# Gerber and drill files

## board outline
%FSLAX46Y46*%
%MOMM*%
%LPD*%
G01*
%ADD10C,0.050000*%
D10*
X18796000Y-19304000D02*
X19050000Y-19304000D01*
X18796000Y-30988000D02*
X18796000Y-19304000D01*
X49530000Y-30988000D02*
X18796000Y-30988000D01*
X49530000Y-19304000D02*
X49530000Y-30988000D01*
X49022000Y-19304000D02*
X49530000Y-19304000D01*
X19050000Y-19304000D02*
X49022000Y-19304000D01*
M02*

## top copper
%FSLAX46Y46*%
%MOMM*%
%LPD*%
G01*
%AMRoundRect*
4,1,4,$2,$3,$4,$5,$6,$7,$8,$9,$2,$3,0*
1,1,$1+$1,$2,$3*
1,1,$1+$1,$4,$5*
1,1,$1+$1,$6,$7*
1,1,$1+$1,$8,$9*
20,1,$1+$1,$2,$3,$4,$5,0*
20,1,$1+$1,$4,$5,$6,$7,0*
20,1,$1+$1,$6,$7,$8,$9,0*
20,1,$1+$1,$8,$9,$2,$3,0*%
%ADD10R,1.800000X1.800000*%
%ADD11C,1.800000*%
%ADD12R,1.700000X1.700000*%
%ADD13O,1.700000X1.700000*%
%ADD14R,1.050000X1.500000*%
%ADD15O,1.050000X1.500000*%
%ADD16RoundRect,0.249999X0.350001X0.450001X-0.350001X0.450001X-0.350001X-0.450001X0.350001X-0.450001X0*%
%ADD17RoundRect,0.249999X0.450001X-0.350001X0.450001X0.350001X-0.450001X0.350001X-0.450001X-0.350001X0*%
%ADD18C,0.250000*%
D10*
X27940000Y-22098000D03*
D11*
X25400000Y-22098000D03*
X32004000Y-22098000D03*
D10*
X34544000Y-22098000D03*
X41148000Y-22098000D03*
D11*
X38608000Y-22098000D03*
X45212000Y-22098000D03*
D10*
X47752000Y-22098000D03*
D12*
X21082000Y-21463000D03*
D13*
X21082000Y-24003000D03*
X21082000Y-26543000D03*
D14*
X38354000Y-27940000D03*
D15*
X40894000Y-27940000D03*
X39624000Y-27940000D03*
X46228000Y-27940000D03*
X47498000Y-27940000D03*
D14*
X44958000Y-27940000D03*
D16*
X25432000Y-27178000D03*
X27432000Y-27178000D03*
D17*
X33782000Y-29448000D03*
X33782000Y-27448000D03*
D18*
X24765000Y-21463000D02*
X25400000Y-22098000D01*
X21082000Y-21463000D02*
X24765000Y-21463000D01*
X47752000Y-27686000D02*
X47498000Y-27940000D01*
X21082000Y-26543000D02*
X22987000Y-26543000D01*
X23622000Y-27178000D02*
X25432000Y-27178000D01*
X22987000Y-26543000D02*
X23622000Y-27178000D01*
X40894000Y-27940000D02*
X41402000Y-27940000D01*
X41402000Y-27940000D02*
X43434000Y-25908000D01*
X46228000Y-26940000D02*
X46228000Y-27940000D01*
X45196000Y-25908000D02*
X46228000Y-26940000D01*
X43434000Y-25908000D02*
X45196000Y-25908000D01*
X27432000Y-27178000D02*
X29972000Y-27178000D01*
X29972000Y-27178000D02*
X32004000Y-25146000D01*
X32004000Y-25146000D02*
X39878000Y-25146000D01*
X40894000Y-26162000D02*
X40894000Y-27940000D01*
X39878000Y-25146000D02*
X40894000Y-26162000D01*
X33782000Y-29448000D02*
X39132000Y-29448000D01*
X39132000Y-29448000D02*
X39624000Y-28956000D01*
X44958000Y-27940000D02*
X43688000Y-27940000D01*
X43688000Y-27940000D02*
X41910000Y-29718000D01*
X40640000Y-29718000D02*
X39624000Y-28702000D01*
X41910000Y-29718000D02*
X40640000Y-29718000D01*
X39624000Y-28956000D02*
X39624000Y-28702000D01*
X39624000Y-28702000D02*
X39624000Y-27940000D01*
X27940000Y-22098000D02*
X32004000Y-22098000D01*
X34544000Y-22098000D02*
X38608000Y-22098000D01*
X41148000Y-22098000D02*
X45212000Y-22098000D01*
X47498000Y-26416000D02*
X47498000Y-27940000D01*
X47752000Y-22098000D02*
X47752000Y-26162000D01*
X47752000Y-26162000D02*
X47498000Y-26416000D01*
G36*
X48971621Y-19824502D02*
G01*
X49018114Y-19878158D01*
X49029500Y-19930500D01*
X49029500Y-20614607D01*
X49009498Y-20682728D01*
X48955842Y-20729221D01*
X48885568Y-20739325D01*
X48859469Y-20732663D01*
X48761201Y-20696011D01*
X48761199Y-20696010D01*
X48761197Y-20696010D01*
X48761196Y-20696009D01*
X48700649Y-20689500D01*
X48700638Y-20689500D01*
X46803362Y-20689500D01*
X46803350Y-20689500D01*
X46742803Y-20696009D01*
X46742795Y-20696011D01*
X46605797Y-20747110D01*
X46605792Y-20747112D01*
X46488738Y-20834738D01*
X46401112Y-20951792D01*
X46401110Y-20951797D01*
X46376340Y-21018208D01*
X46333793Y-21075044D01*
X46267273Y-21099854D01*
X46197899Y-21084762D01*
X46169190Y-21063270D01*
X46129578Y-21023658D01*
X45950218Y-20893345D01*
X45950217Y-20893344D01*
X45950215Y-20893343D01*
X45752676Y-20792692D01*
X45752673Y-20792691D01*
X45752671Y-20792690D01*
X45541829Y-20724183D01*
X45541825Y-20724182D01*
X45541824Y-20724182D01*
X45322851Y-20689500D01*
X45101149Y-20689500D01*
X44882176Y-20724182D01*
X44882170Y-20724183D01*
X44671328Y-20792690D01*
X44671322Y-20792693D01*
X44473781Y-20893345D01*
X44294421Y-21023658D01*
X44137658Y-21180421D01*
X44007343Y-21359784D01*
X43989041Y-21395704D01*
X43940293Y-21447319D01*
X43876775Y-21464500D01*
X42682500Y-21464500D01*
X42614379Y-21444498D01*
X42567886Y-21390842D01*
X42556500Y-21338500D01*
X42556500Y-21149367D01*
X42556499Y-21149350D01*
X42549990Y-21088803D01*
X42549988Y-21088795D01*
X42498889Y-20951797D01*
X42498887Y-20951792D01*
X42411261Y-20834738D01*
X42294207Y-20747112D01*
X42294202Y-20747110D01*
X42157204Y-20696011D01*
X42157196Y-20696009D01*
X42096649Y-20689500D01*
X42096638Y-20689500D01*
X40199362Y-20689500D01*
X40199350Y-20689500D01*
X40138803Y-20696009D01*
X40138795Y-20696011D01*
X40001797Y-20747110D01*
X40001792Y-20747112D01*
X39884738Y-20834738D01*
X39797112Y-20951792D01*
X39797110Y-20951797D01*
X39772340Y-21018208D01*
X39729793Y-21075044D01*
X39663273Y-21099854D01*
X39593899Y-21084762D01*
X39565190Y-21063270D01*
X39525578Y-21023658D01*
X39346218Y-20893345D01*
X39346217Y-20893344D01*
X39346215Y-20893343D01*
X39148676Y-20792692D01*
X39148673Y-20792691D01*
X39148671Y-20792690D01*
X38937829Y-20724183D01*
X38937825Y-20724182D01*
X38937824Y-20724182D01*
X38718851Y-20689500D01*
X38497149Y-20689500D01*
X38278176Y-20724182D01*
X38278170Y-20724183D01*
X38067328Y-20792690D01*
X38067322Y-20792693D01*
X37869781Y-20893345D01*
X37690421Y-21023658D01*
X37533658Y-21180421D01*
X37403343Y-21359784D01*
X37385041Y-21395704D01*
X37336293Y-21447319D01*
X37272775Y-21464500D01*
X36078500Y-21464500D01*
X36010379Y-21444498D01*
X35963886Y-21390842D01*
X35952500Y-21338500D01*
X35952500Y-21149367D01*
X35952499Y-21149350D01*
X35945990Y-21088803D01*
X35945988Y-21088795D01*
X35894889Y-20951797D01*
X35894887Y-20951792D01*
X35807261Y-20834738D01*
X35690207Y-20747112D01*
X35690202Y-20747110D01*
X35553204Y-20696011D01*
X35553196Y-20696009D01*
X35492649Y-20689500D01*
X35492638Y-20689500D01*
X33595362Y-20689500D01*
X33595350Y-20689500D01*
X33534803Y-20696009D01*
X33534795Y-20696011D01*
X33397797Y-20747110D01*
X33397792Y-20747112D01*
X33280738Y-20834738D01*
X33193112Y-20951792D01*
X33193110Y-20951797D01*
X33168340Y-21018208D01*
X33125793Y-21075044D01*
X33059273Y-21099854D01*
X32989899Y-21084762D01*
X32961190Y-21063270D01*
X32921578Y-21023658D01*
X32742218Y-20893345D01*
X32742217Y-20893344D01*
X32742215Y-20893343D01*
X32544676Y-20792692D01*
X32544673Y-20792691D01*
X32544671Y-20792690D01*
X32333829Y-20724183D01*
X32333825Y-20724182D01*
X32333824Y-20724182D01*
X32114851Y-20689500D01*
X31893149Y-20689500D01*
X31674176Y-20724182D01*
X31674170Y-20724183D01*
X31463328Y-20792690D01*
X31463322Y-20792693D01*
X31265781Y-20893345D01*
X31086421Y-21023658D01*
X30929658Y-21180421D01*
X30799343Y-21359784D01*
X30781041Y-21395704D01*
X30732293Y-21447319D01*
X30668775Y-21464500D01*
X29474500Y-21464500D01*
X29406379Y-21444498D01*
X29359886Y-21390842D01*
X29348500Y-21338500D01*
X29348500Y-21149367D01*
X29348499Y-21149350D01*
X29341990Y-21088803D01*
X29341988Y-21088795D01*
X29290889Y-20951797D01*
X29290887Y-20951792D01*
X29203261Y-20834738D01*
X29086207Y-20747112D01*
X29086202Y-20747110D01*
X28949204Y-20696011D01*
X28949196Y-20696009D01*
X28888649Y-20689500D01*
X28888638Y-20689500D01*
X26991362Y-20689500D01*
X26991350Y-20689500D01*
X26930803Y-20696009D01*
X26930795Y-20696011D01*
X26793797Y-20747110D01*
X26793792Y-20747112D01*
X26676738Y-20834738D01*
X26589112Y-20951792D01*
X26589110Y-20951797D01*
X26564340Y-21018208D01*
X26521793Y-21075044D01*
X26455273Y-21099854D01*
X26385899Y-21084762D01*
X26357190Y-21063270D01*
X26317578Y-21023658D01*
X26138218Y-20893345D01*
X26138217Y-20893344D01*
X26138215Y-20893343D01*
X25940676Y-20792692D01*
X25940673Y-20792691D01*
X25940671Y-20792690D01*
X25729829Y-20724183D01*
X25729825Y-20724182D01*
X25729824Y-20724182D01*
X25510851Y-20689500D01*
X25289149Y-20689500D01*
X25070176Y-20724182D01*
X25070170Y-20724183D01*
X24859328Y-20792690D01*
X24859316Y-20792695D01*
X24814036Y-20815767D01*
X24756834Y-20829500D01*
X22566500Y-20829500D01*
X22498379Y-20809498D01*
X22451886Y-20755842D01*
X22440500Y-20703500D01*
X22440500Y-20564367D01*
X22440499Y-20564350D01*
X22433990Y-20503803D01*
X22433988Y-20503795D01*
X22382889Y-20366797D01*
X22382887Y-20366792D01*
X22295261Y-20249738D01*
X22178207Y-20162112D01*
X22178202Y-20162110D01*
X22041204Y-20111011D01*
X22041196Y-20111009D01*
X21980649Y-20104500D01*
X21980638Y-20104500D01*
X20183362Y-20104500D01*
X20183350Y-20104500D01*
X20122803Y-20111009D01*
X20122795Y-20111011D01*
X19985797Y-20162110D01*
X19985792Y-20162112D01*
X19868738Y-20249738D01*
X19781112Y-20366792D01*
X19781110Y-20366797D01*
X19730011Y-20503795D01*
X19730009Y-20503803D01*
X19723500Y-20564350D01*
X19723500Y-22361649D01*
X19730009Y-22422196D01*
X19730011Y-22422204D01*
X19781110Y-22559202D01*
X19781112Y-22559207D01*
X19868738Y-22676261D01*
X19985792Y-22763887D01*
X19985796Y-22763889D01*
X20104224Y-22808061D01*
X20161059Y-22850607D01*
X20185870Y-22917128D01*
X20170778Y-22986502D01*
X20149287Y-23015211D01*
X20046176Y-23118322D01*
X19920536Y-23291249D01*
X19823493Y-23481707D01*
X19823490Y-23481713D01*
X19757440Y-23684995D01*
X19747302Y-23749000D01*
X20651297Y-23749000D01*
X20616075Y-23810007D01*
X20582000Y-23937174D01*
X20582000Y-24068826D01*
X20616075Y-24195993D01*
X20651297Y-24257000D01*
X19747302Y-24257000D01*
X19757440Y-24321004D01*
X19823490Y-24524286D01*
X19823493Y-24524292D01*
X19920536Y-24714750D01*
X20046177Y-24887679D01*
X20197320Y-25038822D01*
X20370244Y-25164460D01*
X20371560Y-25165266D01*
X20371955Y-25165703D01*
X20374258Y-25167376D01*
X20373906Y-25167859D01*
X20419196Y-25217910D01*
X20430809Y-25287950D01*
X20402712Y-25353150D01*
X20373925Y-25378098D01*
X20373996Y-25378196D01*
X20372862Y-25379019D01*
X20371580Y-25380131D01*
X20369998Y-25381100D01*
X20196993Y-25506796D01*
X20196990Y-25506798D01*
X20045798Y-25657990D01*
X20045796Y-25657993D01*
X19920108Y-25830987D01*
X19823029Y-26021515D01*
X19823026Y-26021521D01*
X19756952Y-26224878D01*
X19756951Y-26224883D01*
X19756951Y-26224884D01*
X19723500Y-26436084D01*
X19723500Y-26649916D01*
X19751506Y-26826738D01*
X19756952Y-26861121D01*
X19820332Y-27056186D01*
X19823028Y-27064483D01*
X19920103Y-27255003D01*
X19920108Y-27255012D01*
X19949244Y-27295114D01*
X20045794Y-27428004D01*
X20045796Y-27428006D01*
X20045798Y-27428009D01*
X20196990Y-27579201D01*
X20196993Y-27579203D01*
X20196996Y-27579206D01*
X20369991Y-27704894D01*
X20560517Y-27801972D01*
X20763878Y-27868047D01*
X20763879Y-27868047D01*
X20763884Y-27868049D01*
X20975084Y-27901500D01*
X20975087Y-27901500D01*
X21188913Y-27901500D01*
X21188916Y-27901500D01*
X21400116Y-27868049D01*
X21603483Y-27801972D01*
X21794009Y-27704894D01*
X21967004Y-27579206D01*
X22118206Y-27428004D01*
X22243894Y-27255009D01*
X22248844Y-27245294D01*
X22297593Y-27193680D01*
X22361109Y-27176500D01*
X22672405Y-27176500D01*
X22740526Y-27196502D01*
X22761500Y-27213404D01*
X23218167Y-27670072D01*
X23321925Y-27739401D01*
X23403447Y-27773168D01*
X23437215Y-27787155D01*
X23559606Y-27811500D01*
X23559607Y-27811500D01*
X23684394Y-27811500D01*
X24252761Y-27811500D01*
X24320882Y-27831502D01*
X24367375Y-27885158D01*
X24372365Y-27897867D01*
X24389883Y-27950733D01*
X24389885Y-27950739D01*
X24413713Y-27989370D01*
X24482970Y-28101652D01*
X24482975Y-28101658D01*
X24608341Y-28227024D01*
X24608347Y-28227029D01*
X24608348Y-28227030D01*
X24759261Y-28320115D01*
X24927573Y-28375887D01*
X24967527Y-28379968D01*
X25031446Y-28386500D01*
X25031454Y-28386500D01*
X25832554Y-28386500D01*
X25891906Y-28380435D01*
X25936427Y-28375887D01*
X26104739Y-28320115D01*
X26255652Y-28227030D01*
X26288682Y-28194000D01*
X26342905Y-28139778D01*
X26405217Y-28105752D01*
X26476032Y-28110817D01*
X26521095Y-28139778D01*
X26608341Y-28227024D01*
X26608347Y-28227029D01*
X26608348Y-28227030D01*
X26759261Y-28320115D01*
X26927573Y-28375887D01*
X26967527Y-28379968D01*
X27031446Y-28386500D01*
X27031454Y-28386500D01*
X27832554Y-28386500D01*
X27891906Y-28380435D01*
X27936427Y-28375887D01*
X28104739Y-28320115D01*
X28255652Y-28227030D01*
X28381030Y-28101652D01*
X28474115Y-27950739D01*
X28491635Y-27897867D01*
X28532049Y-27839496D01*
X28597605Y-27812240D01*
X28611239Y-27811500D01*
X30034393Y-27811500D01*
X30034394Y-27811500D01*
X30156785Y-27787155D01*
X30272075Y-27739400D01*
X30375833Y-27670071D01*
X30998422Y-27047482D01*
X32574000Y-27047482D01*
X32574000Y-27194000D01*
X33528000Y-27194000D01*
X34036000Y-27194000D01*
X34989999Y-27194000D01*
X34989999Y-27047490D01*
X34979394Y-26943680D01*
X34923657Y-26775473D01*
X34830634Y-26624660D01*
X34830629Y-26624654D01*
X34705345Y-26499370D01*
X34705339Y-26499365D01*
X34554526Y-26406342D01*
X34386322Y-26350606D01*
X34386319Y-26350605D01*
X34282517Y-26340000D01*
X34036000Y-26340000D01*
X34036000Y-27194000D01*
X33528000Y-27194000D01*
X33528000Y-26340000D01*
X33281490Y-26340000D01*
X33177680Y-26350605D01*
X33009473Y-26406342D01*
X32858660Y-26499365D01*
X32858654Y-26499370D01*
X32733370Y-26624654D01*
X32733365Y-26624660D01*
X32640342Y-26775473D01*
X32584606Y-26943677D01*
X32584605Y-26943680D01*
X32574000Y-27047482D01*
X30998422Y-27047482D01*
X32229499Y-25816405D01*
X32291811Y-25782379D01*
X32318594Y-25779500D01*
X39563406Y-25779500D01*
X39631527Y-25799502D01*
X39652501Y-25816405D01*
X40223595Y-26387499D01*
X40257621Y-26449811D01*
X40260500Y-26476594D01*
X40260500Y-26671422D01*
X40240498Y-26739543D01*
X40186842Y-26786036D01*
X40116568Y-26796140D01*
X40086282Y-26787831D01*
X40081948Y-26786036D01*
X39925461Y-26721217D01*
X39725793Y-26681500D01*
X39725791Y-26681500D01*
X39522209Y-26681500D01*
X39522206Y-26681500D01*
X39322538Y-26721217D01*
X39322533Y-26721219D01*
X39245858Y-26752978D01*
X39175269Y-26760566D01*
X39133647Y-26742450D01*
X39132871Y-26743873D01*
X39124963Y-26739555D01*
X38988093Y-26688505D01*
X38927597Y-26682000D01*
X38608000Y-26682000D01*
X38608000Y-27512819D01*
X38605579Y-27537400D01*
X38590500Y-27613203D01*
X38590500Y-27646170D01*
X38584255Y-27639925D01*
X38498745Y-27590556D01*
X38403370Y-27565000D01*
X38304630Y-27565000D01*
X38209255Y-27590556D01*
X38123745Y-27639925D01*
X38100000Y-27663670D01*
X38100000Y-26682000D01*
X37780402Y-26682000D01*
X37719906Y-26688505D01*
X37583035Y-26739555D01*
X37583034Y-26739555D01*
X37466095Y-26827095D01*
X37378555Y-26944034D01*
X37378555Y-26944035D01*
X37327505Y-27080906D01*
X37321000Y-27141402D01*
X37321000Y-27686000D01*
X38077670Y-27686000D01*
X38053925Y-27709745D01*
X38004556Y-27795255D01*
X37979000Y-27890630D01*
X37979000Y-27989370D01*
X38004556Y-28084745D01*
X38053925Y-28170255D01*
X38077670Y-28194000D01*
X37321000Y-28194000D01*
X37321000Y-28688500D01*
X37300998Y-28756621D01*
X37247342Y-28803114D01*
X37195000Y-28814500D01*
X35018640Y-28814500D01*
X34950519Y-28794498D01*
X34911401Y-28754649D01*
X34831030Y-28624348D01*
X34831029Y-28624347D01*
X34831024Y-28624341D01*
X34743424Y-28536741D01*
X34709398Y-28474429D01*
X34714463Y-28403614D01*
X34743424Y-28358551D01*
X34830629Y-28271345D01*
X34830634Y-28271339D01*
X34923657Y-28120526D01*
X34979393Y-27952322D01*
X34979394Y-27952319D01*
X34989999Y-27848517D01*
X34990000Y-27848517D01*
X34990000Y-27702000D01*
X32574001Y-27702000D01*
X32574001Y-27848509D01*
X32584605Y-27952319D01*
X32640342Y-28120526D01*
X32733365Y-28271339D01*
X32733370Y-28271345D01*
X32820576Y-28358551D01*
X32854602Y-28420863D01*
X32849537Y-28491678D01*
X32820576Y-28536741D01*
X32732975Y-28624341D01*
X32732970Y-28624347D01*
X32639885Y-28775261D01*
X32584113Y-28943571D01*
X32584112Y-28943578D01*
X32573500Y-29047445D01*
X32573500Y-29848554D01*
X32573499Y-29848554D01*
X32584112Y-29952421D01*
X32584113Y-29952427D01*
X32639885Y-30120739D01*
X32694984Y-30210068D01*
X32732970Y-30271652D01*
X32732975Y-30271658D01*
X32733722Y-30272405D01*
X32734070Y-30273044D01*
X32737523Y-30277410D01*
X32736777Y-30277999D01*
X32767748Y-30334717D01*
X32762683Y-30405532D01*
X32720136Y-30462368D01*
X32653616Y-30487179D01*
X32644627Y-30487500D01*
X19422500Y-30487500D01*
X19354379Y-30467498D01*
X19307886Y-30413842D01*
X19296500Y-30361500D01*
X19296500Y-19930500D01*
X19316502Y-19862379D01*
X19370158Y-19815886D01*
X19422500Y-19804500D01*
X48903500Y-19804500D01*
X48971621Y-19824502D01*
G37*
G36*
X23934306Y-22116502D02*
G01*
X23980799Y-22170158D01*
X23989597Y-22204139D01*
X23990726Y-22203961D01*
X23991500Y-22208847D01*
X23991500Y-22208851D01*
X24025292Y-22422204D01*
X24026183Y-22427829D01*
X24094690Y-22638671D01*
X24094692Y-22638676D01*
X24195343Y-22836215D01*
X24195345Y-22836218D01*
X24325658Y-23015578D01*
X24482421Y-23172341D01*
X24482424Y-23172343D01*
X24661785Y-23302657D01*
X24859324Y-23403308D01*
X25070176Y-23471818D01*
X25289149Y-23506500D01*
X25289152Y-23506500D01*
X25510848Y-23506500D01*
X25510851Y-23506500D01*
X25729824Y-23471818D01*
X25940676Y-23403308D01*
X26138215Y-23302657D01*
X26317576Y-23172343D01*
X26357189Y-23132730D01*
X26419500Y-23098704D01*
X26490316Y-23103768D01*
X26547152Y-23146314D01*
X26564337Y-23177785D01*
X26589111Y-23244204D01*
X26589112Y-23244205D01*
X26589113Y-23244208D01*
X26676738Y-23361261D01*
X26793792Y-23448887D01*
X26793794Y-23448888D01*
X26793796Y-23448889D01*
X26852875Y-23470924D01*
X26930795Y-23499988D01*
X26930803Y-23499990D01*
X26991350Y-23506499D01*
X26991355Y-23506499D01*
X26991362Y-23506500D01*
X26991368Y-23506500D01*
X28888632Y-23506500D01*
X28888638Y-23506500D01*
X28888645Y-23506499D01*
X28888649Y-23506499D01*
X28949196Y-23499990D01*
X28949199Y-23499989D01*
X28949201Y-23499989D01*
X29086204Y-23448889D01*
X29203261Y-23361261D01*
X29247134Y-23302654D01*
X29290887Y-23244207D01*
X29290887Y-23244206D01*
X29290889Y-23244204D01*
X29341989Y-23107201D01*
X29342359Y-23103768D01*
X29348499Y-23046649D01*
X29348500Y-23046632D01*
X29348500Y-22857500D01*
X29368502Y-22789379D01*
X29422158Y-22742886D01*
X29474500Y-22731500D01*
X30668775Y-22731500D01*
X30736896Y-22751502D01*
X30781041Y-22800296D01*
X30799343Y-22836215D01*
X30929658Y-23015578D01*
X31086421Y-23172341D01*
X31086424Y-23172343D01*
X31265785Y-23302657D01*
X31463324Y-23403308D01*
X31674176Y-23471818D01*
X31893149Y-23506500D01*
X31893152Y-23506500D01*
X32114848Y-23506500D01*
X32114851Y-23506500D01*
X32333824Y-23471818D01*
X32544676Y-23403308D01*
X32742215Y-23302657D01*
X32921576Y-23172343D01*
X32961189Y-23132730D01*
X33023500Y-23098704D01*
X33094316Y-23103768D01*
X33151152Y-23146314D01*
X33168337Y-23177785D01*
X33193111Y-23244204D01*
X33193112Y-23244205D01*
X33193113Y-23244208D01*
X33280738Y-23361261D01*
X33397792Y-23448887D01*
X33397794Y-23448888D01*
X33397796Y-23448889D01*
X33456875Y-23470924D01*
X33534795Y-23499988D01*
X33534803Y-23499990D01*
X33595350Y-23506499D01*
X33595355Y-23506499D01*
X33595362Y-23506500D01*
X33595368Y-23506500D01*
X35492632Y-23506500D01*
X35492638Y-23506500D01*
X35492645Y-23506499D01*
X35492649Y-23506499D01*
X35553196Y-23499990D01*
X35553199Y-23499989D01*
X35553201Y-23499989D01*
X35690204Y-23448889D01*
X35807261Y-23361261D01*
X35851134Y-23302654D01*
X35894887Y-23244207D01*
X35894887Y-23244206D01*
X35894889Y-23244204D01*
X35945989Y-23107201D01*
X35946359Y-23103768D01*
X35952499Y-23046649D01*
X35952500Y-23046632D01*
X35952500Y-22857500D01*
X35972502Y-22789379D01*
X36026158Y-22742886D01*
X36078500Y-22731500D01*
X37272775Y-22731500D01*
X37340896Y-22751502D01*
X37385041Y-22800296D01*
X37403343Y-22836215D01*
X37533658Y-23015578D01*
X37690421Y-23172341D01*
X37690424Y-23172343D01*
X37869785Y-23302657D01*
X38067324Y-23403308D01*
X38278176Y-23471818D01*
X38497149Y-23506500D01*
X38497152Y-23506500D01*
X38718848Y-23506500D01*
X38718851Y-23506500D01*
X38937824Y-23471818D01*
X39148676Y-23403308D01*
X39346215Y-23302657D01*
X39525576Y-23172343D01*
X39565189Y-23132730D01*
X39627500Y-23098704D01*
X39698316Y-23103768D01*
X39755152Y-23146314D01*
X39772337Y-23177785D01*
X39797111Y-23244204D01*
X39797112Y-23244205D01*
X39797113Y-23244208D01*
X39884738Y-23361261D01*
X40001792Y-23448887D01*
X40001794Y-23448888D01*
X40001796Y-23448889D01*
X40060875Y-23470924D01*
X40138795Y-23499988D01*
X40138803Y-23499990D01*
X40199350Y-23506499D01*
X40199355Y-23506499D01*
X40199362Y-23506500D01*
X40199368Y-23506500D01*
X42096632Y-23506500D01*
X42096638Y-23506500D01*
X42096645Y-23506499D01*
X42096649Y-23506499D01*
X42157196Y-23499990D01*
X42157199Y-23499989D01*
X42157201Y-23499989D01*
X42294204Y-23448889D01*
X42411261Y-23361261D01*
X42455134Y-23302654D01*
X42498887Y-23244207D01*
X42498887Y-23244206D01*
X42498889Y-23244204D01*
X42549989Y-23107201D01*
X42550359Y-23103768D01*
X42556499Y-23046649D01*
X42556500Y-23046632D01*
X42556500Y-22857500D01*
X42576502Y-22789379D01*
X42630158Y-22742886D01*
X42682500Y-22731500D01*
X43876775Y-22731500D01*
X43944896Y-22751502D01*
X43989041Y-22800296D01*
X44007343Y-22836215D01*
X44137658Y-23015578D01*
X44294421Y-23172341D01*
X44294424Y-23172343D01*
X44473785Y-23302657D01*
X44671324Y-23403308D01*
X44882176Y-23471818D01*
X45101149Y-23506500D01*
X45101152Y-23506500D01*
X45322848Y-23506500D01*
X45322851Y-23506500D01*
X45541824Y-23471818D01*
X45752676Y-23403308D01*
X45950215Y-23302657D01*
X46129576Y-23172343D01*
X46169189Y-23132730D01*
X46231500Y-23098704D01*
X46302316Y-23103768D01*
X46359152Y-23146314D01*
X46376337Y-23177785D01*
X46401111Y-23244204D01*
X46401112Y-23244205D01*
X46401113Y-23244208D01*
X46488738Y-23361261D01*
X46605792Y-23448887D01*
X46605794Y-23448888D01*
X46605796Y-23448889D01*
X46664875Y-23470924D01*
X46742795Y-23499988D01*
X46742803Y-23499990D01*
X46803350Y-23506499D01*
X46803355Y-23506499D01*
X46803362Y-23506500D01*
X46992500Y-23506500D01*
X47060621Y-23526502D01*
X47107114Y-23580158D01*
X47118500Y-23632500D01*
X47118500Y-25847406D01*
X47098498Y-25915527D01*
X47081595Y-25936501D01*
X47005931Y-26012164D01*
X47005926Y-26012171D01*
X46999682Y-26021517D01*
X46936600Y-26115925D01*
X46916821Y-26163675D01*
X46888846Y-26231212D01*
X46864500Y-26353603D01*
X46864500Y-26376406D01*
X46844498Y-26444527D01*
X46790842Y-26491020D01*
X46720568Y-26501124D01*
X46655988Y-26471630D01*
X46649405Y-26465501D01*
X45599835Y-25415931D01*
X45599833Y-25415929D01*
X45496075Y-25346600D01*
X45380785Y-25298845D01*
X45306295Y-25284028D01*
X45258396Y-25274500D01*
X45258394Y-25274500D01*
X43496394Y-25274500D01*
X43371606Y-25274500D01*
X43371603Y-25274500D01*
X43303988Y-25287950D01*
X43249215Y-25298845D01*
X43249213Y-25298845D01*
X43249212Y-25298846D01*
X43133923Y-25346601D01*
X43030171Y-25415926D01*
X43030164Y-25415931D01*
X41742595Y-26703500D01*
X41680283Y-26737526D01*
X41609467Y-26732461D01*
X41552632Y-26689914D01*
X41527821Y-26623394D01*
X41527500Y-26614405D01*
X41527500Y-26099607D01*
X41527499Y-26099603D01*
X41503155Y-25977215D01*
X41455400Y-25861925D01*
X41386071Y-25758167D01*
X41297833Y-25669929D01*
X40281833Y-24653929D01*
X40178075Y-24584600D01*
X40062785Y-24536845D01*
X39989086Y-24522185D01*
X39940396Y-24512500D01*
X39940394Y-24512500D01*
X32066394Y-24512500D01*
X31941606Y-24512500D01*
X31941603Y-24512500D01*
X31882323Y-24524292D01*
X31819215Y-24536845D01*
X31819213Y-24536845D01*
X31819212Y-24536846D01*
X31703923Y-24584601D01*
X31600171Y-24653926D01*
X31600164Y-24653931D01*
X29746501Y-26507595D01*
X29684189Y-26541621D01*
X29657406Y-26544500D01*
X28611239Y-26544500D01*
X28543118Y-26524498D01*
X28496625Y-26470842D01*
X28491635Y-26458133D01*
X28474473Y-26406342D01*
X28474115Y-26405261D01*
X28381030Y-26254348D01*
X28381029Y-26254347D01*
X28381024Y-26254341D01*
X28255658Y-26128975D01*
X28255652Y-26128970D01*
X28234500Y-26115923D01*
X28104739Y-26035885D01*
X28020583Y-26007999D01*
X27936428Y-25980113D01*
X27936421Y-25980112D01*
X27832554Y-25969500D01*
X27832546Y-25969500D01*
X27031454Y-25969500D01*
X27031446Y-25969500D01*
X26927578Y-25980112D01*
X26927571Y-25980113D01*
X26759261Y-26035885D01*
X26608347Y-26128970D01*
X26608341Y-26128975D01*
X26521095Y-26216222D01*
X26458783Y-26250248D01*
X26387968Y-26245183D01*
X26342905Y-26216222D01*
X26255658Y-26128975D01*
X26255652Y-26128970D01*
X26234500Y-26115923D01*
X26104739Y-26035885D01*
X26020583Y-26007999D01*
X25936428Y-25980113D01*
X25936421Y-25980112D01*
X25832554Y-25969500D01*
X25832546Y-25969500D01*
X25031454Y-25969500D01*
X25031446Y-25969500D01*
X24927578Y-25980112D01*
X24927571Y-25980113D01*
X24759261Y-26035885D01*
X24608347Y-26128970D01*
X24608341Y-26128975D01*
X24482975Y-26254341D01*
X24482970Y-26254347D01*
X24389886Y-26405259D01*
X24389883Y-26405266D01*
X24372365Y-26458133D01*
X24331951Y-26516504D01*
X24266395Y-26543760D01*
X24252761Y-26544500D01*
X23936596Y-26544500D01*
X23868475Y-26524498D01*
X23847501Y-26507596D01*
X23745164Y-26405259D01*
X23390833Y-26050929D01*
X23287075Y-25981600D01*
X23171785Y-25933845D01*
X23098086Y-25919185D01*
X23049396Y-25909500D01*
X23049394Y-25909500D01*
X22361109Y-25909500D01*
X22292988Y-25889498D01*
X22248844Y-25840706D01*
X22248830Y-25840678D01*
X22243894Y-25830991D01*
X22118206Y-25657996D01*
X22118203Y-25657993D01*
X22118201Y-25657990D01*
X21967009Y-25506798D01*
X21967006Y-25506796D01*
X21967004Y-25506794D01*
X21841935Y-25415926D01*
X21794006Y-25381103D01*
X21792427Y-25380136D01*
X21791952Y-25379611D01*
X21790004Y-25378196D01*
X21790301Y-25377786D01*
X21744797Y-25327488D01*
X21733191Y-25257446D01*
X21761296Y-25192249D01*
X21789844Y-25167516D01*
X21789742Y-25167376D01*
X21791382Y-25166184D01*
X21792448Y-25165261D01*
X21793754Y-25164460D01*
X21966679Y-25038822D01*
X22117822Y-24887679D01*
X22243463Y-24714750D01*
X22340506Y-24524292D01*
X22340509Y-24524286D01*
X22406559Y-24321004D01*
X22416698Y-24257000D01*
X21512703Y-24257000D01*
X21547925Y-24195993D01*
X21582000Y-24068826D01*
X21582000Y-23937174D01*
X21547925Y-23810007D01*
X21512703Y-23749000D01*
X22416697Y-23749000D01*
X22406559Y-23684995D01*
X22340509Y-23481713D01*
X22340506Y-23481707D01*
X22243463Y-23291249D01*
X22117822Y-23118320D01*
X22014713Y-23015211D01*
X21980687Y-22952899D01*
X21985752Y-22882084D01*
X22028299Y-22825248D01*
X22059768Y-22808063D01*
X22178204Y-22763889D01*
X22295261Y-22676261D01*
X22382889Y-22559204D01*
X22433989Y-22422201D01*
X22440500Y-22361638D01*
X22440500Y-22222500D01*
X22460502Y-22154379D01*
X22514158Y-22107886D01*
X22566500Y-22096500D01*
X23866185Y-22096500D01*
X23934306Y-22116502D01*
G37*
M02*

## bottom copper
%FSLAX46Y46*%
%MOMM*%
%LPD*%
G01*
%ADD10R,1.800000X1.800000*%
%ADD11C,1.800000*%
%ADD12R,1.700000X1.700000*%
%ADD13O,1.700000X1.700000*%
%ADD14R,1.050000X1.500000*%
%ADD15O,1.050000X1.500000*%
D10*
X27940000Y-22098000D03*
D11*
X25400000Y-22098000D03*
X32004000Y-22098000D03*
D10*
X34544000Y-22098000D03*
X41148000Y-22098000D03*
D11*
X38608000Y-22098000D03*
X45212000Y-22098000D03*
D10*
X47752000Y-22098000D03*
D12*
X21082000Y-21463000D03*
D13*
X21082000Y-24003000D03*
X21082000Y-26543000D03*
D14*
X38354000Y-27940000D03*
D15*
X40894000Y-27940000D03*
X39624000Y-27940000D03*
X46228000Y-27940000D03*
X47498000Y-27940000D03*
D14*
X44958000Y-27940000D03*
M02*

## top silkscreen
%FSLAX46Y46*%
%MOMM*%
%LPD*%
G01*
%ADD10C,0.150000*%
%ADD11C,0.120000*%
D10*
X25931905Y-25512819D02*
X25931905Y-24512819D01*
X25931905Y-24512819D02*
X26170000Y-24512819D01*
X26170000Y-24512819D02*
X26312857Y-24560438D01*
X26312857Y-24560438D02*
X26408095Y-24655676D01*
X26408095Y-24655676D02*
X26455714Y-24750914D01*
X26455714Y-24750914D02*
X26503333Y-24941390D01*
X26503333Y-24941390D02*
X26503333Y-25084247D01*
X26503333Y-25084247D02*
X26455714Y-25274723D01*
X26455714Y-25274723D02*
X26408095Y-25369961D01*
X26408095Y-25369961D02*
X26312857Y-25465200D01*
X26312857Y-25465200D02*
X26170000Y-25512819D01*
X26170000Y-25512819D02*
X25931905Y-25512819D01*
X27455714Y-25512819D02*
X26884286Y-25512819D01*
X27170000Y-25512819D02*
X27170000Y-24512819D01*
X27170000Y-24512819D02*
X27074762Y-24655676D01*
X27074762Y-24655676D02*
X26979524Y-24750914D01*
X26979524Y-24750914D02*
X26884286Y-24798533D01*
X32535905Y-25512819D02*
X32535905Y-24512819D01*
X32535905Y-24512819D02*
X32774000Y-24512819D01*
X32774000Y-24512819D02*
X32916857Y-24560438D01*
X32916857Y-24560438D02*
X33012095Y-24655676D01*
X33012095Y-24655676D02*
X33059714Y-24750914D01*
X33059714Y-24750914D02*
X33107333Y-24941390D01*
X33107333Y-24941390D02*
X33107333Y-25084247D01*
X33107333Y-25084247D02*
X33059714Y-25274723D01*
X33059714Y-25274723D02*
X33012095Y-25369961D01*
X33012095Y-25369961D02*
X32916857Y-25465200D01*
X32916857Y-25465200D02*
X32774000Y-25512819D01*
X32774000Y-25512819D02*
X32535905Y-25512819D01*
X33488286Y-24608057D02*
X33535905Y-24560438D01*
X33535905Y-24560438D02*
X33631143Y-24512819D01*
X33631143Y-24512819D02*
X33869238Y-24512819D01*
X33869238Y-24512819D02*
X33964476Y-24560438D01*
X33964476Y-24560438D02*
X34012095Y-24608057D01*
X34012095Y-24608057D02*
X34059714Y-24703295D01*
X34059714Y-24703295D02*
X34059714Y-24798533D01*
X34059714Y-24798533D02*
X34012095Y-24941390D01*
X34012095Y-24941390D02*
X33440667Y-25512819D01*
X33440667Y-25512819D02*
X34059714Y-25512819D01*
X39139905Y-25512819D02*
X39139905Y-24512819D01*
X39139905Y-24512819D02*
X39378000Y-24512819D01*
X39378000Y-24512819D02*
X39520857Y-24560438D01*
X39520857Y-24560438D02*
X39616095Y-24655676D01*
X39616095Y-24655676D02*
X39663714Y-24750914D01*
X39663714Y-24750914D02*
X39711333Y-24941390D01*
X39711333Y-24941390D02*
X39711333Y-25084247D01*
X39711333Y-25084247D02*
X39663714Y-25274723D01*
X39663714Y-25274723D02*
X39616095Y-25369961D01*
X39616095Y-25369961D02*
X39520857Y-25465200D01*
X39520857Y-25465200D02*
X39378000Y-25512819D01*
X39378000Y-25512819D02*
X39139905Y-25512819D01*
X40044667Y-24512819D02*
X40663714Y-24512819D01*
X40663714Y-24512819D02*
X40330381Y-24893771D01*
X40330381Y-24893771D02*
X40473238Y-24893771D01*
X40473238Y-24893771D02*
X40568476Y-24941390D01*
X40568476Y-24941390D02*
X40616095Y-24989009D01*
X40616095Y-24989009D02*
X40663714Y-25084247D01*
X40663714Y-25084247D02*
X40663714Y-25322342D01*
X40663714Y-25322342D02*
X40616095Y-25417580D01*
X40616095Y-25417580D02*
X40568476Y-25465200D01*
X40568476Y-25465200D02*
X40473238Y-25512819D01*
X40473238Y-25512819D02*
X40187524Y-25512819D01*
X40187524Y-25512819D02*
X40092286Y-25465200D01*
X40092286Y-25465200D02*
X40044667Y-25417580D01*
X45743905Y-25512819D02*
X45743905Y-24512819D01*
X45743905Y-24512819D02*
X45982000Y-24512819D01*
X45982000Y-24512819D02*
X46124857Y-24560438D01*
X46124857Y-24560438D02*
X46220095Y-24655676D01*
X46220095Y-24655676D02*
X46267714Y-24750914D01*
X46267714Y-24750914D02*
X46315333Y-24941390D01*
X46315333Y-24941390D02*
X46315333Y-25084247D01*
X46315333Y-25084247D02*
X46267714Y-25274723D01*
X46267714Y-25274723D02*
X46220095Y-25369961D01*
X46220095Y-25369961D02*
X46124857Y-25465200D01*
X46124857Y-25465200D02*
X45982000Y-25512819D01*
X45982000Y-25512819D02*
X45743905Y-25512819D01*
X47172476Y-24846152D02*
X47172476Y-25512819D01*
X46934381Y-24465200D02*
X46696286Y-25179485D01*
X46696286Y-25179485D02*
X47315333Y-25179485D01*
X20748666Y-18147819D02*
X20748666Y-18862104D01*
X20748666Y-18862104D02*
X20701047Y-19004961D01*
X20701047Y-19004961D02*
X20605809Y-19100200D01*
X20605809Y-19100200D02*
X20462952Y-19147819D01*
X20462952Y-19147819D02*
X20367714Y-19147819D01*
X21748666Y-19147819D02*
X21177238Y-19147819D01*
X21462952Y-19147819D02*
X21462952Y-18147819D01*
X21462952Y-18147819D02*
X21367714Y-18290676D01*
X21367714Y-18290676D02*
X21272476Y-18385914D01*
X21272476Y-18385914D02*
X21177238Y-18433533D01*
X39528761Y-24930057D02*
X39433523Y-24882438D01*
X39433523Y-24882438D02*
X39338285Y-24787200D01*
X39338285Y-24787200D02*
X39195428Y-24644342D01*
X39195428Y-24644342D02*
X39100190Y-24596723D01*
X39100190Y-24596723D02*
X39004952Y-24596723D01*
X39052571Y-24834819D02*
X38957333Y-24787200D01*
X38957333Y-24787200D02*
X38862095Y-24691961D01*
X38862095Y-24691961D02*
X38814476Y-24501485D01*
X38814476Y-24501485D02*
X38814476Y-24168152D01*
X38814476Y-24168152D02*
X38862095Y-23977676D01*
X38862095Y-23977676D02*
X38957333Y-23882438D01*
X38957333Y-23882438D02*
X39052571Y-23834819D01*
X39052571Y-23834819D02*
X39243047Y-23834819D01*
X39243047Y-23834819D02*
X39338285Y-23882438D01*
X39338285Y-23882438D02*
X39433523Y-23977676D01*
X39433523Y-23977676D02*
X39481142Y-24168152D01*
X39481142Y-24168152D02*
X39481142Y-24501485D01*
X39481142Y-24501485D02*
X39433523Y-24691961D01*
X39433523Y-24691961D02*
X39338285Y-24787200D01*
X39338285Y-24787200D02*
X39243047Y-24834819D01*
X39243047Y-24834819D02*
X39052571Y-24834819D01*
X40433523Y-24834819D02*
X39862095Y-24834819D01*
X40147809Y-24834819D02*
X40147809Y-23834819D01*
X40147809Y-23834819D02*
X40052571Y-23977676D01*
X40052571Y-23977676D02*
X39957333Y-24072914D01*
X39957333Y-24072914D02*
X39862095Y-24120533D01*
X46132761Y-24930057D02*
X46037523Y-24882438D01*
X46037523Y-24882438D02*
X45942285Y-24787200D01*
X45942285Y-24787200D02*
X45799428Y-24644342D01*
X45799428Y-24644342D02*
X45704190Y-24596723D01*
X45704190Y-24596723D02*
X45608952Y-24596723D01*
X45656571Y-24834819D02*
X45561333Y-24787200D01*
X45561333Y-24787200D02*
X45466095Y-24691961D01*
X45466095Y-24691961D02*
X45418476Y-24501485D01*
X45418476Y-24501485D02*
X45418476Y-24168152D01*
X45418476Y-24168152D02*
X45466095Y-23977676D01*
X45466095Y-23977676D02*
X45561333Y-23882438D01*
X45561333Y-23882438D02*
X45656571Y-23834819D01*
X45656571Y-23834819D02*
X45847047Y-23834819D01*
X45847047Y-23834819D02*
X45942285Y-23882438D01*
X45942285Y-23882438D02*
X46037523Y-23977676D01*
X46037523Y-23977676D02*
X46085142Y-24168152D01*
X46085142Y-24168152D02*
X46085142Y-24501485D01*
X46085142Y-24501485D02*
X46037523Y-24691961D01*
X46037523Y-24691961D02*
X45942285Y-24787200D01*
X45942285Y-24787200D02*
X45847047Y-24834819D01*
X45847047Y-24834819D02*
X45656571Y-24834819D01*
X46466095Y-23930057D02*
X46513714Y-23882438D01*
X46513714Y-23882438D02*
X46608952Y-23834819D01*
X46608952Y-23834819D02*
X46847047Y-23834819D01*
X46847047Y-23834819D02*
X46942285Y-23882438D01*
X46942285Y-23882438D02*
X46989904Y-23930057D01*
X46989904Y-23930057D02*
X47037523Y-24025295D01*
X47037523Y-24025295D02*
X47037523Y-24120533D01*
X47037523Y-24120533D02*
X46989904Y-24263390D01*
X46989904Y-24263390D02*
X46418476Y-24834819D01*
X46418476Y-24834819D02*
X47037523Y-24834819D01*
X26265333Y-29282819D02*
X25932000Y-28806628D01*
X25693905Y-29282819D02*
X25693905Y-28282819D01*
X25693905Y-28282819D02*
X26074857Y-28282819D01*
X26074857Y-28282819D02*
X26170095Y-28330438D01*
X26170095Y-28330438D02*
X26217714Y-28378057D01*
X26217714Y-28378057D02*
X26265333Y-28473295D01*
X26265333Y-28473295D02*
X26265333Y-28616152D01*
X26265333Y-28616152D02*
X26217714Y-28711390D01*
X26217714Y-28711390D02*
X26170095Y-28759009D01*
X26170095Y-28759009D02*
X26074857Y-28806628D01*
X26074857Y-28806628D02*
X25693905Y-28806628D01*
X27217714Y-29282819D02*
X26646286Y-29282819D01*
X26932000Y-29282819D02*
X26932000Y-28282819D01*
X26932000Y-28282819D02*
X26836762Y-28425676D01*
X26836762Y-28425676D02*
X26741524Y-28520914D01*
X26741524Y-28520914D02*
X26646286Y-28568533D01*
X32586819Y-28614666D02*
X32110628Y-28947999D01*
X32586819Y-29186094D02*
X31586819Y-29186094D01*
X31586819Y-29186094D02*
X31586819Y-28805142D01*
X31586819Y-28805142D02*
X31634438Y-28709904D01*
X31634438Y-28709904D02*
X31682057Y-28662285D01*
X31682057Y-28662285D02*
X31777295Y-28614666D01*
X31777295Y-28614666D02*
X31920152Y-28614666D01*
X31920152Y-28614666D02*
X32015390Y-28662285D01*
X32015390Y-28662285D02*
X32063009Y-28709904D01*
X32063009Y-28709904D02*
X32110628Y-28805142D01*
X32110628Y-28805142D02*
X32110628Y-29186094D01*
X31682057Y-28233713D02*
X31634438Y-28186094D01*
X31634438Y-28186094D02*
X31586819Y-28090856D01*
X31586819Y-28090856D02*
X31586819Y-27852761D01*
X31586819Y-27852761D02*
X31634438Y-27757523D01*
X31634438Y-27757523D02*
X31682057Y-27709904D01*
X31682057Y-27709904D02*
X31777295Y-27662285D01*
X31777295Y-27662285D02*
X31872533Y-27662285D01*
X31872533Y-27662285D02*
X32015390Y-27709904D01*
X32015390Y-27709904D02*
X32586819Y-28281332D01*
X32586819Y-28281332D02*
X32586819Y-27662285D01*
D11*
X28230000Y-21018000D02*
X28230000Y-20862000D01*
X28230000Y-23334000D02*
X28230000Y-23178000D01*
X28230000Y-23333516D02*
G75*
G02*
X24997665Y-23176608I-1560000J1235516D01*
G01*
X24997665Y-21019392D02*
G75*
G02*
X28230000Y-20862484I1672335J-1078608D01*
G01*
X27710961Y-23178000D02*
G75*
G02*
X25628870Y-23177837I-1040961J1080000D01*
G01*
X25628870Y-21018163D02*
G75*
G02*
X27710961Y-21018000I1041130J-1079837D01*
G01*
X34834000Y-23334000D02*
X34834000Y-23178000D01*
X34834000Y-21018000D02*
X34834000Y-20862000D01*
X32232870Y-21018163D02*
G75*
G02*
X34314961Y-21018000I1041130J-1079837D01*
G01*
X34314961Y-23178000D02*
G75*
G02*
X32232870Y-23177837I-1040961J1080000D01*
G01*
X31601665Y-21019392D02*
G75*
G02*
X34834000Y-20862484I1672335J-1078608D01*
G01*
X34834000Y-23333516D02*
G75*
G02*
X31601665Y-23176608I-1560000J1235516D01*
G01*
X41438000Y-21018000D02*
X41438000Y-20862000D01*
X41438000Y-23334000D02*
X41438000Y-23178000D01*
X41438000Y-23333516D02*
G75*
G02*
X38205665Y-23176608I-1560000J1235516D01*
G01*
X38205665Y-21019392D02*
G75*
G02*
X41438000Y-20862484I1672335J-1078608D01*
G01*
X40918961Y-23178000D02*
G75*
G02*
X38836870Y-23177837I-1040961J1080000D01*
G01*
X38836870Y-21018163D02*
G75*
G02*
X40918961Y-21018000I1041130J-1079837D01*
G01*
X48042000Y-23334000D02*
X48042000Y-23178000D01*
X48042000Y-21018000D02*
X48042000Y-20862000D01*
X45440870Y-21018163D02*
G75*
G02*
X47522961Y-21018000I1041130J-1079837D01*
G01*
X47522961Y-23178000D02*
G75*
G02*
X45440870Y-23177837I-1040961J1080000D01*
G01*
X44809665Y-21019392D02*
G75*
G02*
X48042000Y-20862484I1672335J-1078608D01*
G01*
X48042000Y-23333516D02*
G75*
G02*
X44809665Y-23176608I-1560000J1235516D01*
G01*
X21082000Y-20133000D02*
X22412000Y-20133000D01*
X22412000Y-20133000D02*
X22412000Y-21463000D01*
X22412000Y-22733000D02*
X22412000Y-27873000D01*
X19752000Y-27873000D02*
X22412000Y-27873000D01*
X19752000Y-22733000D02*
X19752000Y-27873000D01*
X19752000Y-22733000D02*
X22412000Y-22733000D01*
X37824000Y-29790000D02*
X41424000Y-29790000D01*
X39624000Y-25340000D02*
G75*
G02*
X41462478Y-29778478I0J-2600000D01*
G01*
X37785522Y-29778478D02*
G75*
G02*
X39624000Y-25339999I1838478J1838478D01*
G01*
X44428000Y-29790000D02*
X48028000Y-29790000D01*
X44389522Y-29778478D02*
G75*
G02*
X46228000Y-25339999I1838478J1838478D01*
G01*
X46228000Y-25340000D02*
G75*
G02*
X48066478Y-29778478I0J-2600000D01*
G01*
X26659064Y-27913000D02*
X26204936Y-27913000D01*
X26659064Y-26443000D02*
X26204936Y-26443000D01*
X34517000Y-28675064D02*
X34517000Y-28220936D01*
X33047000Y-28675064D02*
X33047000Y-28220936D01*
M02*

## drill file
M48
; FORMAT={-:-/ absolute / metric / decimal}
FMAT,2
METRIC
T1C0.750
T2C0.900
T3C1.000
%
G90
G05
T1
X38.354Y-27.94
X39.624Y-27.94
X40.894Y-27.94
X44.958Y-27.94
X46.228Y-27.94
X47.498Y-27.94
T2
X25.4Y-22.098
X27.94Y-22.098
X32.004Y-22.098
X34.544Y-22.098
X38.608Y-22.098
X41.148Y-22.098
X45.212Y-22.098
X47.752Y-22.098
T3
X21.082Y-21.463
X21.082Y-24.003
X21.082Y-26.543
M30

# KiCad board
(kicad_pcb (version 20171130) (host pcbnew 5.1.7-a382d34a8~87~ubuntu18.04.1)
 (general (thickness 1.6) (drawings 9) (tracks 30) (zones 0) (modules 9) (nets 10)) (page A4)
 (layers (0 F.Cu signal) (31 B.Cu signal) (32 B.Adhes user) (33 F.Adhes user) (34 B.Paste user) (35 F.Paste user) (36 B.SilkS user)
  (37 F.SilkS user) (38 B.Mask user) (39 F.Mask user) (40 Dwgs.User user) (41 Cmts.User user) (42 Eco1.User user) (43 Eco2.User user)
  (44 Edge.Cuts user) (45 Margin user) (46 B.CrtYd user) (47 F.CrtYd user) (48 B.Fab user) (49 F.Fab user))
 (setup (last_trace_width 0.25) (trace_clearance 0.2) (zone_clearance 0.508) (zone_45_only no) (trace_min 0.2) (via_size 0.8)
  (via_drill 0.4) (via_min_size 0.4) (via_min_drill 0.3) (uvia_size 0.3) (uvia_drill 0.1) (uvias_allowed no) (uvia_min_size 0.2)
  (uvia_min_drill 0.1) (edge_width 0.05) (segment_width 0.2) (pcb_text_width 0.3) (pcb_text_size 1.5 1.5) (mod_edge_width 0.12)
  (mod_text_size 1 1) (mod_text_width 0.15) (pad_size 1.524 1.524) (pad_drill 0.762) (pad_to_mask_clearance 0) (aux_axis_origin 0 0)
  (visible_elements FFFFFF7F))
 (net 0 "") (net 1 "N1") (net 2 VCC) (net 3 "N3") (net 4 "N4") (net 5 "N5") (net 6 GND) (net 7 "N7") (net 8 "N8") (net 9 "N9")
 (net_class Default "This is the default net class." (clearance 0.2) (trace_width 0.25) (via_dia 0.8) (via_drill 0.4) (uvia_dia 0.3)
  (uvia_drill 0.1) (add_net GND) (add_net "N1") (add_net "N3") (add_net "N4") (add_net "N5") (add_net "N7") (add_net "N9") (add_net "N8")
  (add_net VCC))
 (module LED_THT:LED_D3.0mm (layer F.Cu) (at 27.94 22.098 180)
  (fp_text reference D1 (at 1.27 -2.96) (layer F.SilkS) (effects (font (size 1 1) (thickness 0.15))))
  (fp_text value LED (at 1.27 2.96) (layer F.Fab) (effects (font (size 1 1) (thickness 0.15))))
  (fp_line (start -0.29 1.08) (end -0.29 1.236) (layer F.SilkS) (width 0.12))
  (fp_line (start -0.29 -1.236) (end -0.29 -1.08) (layer F.SilkS) (width 0.12))
  (fp_arc (start 1.27 0) (end -0.29 -1.235516) (angle 108.8) (layer F.SilkS) (width 0.12))
  (fp_arc (start 1.27 0) (end -0.29 1.235516) (angle -108.8) (layer F.SilkS) (width 0.12))
  (fp_arc (start 1.27 0) (end 0.229039 -1.08) (angle 87.9) (layer F.SilkS) (width 0.12))
  (fp_arc (start 1.27 0) (end 0.229039 1.08) (angle -87.9) (layer F.SilkS) (width 0.12))
  (pad 1 thru_hole rect (at 0 0 180) (size 1.8 1.8) (drill 0.9) (layers *.Cu *.Mask) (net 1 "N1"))
  (pad 2 thru_hole circle (at 2.54 0 180) (size 1.8 1.8) (drill 0.9) (layers *.Cu *.Mask) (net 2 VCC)))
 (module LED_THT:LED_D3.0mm (layer F.Cu) (at 34.544 22.098 180)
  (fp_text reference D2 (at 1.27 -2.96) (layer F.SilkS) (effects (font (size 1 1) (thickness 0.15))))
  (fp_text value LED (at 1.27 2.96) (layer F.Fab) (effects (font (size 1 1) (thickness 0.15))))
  (fp_line (start -0.29 -1.236) (end -0.29 -1.08) (layer F.SilkS) (width 0.12))
  (fp_line (start -0.29 1.08) (end -0.29 1.236) (layer F.SilkS) (width 0.12))
  (fp_arc (start 1.27 0) (end 0.229039 1.08) (angle -87.9) (layer F.SilkS) (width 0.12))
  (fp_arc (start 1.27 0) (end 0.229039 -1.08) (angle 87.9) (layer F.SilkS) (width 0.12))
  (fp_arc (start 1.27 0) (end -0.29 1.235516) (angle -108.8) (layer F.SilkS) (width 0.12))
  (fp_arc (start 1.27 0) (end -0.29 -1.235516) (angle 108.8) (layer F.SilkS) (width 0.12))
  (pad 2 thru_hole circle (at 2.54 0 180) (size 1.8 1.8) (drill 0.9) (layers *.Cu *.Mask) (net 1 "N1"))
  (pad 1 thru_hole rect (at 0 0 180) (size 1.8 1.8) (drill 0.9) (layers *.Cu *.Mask) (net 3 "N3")))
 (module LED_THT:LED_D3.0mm (layer F.Cu) (at 41.148 22.098 180)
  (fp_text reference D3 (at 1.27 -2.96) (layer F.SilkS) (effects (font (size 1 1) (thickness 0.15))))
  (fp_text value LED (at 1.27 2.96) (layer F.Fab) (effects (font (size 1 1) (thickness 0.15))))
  (fp_line (start -0.29 1.08) (end -0.29 1.236) (layer F.SilkS) (width 0.12))
  (fp_line (start -0.29 -1.236) (end -0.29 -1.08) (layer F.SilkS) (width 0.12))
  (fp_arc (start 1.27 0) (end -0.29 -1.235516) (angle 108.8) (layer F.SilkS) (width 0.12))
  (fp_arc (start 1.27 0) (end -0.29 1.235516) (angle -108.8) (layer F.SilkS) (width 0.12))
  (fp_arc (start 1.27 0) (end 0.229039 -1.08) (angle 87.9) (layer F.SilkS) (width 0.12))
  (fp_arc (start 1.27 0) (end 0.229039 1.08) (angle -87.9) (layer F.SilkS) (width 0.12))
  (pad 1 thru_hole rect (at 0 0 180) (size 1.8 1.8) (drill 0.9) (layers *.Cu *.Mask) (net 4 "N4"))
  (pad 2 thru_hole circle (at 2.54 0 180) (size 1.8 1.8) (drill 0.9) (layers *.Cu *.Mask) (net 3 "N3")))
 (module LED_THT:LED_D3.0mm (layer F.Cu) (at 47.752 22.098 180)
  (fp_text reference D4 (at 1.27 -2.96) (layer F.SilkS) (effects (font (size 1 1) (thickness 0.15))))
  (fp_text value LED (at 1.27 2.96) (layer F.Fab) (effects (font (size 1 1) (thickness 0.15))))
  (fp_line (start -0.29 -1.236) (end -0.29 -1.08) (layer F.SilkS) (width 0.12))
  (fp_line (start -0.29 1.08) (end -0.29 1.236) (layer F.SilkS) (width 0.12))
  (fp_arc (start 1.27 0) (end 0.229039 1.08) (angle -87.9) (layer F.SilkS) (width 0.12))
  (fp_arc (start 1.27 0) (end 0.229039 -1.08) (angle 87.9) (layer F.SilkS) (width 0.12))
  (fp_arc (start 1.27 0) (end -0.29 1.235516) (angle -108.8) (layer F.SilkS) (width 0.12))
  (fp_arc (start 1.27 0) (end -0.29 -1.235516) (angle 108.8) (layer F.SilkS) (width 0.12))
  (pad 2 thru_hole circle (at 2.54 0 180) (size 1.8 1.8) (drill 0.9) (layers *.Cu *.Mask) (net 4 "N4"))
  (pad 1 thru_hole rect (at 0 0 180) (size 1.8 1.8) (drill 0.9) (layers *.Cu *.Mask) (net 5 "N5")))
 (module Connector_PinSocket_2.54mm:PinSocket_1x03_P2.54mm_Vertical (layer F.Cu) (at 21.082 21.463)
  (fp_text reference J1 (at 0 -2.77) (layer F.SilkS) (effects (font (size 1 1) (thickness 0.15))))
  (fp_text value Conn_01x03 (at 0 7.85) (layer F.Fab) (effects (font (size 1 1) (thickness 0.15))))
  (fp_line (start 0 -1.33) (end 1.33 -1.33) (layer F.SilkS) (width 0.12))
  (fp_line (start 1.33 -1.33) (end 1.33 0) (layer F.SilkS) (width 0.12))
  (fp_line (start 1.33 1.27) (end 1.33 6.41) (layer F.SilkS) (width 0.12))
  (fp_line (start -1.33 6.41) (end 1.33 6.41) (layer F.SilkS) (width 0.12))
  (fp_line (start -1.33 1.27) (end -1.33 6.41) (layer F.SilkS) (width 0.12))
  (fp_line (start -1.33 1.27) (end 1.33 1.27) (layer F.SilkS) (width 0.12))
  (pad 1 thru_hole rect (at 0 0) (size 1.7 1.7) (drill 1) (layers *.Cu *.Mask) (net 2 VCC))
  (pad 2 thru_hole oval (at 0 2.54) (size 1.7 1.7) (drill 1) (layers *.Cu *.Mask) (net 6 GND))
  (pad 3 thru_hole oval (at 0 5.08) (size 1.7 1.7) (drill 1) (layers *.Cu *.Mask) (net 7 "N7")))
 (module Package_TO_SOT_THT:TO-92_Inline (layer F.Cu) (at 38.354 27.94)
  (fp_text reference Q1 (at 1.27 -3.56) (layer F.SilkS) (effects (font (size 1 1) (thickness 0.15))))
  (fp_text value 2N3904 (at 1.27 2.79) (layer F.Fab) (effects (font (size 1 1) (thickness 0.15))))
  (fp_line (start -0.53 1.85) (end 3.07 1.85) (layer F.SilkS) (width 0.12))
  (fp_arc (start 1.27 0) (end 1.27 -2.6) (angle 135) (layer F.SilkS) (width 0.12))
  (fp_arc (start 1.27 0) (end 1.27 -2.6) (angle -135) (layer F.SilkS) (width 0.12))
  (pad 1 thru_hole rect (at 0 0) (size 1.05 1.5) (drill 0.75) (layers *.Cu *.Mask) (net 6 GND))
  (pad 3 thru_hole oval (at 2.54 0) (size 1.05 1.5) (drill 0.75) (layers *.Cu *.Mask) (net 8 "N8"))
  (pad 2 thru_hole oval (at 1.27 0) (size 1.05 1.5) (drill 0.75) (layers *.Cu *.Mask) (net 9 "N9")))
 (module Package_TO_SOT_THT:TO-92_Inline (layer F.Cu) (at 44.958 27.94)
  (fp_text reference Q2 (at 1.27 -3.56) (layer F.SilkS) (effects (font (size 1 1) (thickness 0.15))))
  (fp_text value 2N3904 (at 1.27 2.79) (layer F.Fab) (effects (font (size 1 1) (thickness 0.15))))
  (fp_line (start -0.53 1.85) (end 3.07 1.85) (layer F.SilkS) (width 0.12))
  (fp_arc (start 1.27 0) (end 1.27 -2.6) (angle -135) (layer F.SilkS) (width 0.12))
  (fp_arc (start 1.27 0) (end 1.27 -2.6) (angle 135) (layer F.SilkS) (width 0.12))
  (pad 2 thru_hole oval (at 1.27 0) (size 1.05 1.5) (drill 0.75) (layers *.Cu *.Mask) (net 8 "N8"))
  (pad 3 thru_hole oval (at 2.54 0) (size 1.05 1.5) (drill 0.75) (layers *.Cu *.Mask) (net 5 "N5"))
  (pad 1 thru_hole rect (at 0 0) (size 1.05 1.5) (drill 0.75) (layers *.Cu *.Mask) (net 9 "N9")))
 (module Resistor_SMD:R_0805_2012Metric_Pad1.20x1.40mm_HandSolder (layer F.Cu) (at 26.432 27.178 180)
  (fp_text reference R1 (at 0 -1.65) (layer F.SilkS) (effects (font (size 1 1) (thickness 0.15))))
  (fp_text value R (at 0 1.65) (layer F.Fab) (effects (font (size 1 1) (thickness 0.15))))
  (fp_line (start -0.227064 -0.735) (end 0.227064 -0.735) (layer F.SilkS) (width 0.12))
  (fp_line (start -0.227064 0.735) (end 0.227064 0.735) (layer F.SilkS) (width 0.12))
  (pad 2 smd roundrect (at 1 0 180) (size 1.2 1.4) (layers F.Cu F.Paste F.Mask) (roundrect_rratio 0.2083325) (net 7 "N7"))
  (pad 1 smd roundrect (at -1 0 180) (size 1.2 1.4) (layers F.Cu F.Paste F.Mask) (roundrect_rratio 0.2083325) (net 8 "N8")))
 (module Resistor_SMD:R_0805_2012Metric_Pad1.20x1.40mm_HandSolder (layer F.Cu) (at 33.782 28.448 90)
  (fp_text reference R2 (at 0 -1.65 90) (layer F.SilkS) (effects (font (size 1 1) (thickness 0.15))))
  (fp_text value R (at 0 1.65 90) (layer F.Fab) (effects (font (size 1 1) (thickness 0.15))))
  (fp_line (start -0.227064 0.735) (end 0.227064 0.735) (layer F.SilkS) (width 0.12))
  (fp_line (start -0.227064 -0.735) (end 0.227064 -0.735) (layer F.SilkS) (width 0.12))
  (pad 1 smd roundrect (at -1 0 90) (size 1.2 1.4) (layers F.Cu F.Paste F.Mask) (roundrect_rratio 0.2083325) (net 9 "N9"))
  (pad 2 smd roundrect (at 1 0 90) (size 1.2 1.4) (layers F.Cu F.Paste F.Mask) (roundrect_rratio 0.2083325) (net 6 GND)))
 (gr_line (start 18.796 19.304) (end 19.05 19.304) (layer Edge.Cuts) (width 0.05))
 (gr_line (start 18.796 30.988) (end 18.796 19.304) (layer Edge.Cuts) (width 0.05))
 (gr_line (start 49.53 30.988) (end 18.796 30.988) (layer Edge.Cuts) (width 0.05))
 (gr_line (start 49.53 19.304) (end 49.53 30.988) (layer Edge.Cuts) (width 0.05))
 (gr_line (start 49.022 19.304) (end 49.53 19.304) (layer Edge.Cuts) (width 0.05))
 (gr_line (start 19.05 19.304) (end 49.022 19.304) (layer Edge.Cuts) (width 0.05))
 (segment (start 24.765 21.463) (end 25.4 22.098) (width 0.25) (layer F.Cu) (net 2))
 (segment (start 21.082 21.463) (end 24.765 21.463) (width 0.25) (layer F.Cu) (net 2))
 (segment (start 47.752 27.686) (end 47.498 27.94) (width 0.25) (layer F.Cu) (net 5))
 (segment (start 21.082 26.543) (end 22.987 26.543) (width 0.25) (layer F.Cu) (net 7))
 (segment (start 23.622 27.178) (end 25.432 27.178) (width 0.25) (layer F.Cu) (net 7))
 (segment (start 22.987 26.543) (end 23.622 27.178) (width 0.25) (layer F.Cu) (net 7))
 (segment (start 40.894 27.94) (end 41.402 27.94) (width 0.25) (layer F.Cu) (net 8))
 (segment (start 41.402 27.94) (end 43.434 25.908) (width 0.25) (layer F.Cu) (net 8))
 (segment (start 46.228 26.94) (end 46.228 27.94) (width 0.25) (layer F.Cu) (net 8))
 (segment (start 45.196 25.908) (end 46.228 26.94) (width 0.25) (layer F.Cu) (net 8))
 (segment (start 43.434 25.908) (end 45.196 25.908) (width 0.25) (layer F.Cu) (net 8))
 (segment (start 27.432 27.178) (end 29.972 27.178) (width 0.25) (layer F.Cu) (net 8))
 (segment (start 29.972 27.178) (end 32.004 25.146) (width 0.25) (layer F.Cu) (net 8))
 (segment (start 32.004 25.146) (end 39.878 25.146) (width 0.25) (layer F.Cu) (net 8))
 (segment (start 40.894 26.162) (end 40.894 27.94) (width 0.25) (layer F.Cu) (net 8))
 (segment (start 39.878 25.146) (end 40.894 26.162) (width 0.25) (layer F.Cu) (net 8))
 (segment (start 33.782 29.448) (end 39.132 29.448) (width 0.25) (layer F.Cu) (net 9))
 (segment (start 39.132 29.448) (end 39.624 28.956) (width 0.25) (layer F.Cu) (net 9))
 (segment (start 44.958 27.94) (end 43.688 27.94) (width 0.25) (layer F.Cu) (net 9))
 (segment (start 43.688 27.94) (end 41.91 29.718) (width 0.25) (layer F.Cu) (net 9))
 (segment (start 40.64 29.718) (end 39.624 28.702) (width 0.25) (layer F.Cu) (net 9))
 (segment (start 41.91 29.718) (end 40.64 29.718) (width 0.25) (layer F.Cu) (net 9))
 (segment (start 39.624 28.956) (end 39.624 28.702) (width 0.25) (layer F.Cu) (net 9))
 (segment (start 39.624 28.702) (end 39.624 27.94) (width 0.25) (layer F.Cu) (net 9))
 (segment (start 27.94 22.098) (end 32.004 22.098) (width 0.25) (layer F.Cu) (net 1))
 (segment (start 34.544 22.098) (end 38.608 22.098) (width 0.25) (layer F.Cu) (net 3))
 (segment (start 41.148 22.098) (end 45.212 22.098) (width 0.25) (layer F.Cu) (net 4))
 (segment (start 47.498 26.416) (end 47.498 27.94) (width 0.25) (layer F.Cu) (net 5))
 (segment (start 47.752 22.098) (end 47.752 26.162) (width 0.25) (layer F.Cu) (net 5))
 (segment (start 47.752 26.162) (end 47.498 26.416) (width 0.25) (layer F.Cu) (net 5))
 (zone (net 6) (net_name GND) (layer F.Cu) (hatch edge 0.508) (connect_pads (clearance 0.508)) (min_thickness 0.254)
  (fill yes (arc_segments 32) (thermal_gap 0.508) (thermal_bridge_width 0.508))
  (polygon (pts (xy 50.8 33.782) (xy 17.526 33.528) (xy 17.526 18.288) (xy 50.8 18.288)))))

